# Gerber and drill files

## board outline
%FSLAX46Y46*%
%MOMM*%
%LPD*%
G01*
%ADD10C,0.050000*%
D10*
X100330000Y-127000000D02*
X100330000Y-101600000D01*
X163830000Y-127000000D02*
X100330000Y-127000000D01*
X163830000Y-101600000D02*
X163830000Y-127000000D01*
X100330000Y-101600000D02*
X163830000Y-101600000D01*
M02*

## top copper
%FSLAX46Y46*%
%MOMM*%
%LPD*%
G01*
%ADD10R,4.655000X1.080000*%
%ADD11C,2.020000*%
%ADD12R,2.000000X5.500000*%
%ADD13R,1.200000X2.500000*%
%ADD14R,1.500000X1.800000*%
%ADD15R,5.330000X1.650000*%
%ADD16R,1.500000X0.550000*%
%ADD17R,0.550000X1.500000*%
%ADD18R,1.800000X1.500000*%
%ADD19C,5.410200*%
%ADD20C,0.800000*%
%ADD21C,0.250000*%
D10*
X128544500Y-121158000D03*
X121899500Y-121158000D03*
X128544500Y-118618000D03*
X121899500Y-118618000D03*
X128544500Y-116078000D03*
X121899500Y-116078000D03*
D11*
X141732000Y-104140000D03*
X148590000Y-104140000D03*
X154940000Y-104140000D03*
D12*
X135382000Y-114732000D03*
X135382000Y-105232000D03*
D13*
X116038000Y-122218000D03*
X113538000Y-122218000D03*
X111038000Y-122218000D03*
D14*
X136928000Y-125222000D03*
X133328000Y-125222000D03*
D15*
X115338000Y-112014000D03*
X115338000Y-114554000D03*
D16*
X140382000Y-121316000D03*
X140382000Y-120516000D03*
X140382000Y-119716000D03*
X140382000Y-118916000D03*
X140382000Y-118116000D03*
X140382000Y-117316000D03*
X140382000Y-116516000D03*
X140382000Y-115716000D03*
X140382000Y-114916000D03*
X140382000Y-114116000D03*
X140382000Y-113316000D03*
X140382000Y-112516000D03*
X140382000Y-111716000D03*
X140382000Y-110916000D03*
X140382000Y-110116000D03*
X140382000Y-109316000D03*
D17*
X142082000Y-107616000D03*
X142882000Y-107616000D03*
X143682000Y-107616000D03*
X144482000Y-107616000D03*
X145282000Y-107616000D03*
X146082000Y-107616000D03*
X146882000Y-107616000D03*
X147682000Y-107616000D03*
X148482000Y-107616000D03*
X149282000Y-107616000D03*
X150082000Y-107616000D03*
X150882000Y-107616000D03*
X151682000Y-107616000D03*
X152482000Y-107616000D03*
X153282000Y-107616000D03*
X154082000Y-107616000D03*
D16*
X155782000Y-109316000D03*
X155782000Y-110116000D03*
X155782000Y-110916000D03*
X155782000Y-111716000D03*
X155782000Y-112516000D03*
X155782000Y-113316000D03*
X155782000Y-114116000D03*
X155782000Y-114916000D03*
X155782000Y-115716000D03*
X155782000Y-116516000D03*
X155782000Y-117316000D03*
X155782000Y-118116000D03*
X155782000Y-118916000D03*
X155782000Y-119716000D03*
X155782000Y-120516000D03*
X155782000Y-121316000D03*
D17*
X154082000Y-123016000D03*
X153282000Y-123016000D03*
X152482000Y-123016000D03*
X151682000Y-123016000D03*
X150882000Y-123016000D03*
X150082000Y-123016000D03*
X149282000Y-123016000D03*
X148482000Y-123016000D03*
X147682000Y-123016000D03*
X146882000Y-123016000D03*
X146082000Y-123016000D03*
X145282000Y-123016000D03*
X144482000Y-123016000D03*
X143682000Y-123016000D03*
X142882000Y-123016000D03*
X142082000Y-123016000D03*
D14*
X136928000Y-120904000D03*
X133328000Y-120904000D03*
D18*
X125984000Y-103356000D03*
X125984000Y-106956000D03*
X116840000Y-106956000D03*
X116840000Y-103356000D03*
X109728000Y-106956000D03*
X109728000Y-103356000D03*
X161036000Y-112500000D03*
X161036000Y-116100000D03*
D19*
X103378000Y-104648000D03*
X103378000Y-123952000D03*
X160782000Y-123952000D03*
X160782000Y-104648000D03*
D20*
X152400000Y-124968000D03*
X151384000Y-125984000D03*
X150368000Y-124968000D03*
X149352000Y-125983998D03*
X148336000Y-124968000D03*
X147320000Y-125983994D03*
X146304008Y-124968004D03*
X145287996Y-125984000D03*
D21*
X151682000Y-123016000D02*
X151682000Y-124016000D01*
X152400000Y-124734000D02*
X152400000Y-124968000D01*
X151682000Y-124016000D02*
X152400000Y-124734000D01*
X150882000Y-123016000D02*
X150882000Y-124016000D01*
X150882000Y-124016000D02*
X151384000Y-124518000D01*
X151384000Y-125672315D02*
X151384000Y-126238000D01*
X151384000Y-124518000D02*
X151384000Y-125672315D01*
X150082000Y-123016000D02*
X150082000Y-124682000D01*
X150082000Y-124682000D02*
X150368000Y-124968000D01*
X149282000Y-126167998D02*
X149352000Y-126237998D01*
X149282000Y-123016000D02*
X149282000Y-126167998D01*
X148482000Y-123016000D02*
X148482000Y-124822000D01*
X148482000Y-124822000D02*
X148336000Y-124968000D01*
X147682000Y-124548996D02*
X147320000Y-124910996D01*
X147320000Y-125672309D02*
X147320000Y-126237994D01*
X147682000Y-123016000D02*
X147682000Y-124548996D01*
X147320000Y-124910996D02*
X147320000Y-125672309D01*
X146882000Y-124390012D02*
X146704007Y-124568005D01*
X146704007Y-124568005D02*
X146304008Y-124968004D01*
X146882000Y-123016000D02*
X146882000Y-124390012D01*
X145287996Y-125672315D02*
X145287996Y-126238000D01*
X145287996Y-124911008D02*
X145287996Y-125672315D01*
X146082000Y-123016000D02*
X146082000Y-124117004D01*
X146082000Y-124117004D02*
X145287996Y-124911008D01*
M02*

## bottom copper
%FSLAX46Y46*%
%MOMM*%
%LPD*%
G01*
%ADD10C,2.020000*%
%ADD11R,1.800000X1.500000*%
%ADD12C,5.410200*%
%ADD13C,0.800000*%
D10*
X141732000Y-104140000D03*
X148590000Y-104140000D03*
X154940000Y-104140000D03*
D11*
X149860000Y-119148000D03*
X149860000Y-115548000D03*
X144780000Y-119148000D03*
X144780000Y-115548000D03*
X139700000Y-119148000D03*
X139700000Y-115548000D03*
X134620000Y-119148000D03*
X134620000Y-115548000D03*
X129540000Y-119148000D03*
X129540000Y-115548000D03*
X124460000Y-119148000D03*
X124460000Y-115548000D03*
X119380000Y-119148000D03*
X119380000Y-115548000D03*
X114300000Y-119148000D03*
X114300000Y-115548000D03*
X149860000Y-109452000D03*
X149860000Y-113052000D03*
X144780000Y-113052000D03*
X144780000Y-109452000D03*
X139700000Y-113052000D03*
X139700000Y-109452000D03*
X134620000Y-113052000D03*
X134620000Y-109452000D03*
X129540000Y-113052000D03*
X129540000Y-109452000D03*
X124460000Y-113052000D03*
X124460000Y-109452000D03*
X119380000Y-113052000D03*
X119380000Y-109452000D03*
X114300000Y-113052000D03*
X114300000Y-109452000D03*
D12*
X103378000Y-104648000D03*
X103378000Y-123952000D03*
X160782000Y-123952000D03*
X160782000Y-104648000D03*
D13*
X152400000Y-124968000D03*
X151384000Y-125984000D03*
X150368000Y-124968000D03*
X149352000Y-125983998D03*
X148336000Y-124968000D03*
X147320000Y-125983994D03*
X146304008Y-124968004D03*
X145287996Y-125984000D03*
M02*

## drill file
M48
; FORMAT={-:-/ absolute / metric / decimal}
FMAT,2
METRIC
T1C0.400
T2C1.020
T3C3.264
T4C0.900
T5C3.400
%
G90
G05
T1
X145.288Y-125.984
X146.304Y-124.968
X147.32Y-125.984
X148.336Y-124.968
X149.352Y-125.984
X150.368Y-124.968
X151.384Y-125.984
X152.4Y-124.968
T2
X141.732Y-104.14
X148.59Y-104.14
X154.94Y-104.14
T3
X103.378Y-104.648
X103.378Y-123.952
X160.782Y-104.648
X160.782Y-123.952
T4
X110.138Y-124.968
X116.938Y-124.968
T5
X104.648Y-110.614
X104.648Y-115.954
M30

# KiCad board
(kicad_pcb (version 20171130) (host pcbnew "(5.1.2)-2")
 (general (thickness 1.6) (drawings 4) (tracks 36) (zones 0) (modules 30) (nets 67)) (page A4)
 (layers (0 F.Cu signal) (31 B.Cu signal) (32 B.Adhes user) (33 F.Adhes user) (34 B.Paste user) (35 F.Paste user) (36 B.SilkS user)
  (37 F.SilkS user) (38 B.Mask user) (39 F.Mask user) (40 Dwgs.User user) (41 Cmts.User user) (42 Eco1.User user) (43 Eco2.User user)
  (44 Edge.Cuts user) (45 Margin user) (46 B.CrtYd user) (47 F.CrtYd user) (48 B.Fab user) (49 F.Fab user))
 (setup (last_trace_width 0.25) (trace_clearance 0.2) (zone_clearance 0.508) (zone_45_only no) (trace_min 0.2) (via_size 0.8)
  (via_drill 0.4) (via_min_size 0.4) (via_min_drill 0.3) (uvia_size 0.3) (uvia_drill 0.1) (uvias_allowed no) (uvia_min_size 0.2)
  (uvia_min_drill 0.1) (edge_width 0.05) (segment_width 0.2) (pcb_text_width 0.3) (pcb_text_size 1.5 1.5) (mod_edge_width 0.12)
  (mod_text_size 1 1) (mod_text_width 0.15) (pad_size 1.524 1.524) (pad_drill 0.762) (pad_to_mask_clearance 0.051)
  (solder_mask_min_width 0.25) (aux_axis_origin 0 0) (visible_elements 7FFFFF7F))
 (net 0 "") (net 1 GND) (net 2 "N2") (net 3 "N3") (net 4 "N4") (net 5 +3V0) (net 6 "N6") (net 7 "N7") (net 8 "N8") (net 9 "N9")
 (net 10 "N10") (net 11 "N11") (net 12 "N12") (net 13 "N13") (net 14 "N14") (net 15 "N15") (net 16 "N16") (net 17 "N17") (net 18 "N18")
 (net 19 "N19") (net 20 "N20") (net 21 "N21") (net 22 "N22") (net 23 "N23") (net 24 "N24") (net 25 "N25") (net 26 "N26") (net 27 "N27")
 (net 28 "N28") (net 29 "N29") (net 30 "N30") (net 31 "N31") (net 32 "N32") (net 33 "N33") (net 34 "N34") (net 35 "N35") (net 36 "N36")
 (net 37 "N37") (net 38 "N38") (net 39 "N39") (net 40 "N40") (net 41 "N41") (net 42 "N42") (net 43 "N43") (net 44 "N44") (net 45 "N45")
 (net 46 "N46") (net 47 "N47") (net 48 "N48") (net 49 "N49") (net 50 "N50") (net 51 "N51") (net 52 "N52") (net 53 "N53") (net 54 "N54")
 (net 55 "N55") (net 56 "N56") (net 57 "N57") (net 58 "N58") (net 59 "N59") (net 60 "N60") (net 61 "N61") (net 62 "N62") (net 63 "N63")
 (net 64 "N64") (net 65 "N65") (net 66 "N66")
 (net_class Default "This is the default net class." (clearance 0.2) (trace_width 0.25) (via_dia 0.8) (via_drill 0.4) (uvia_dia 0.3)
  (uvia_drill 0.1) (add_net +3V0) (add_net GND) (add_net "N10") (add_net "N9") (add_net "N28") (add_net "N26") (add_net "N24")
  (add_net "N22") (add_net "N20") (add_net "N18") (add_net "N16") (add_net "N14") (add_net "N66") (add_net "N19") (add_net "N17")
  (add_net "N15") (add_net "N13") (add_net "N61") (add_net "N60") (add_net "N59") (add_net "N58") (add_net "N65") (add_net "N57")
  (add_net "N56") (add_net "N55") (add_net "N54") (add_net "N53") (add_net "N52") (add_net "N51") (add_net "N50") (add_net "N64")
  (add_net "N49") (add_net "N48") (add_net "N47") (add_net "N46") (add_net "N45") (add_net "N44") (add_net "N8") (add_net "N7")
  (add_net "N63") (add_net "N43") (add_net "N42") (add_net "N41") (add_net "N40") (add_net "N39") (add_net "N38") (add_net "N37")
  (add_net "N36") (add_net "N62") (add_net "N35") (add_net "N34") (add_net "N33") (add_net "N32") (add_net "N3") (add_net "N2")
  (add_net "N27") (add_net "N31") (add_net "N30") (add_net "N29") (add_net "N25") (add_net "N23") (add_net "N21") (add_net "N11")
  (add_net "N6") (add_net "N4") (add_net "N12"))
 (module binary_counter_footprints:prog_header (layer F.Cu) (at 125.222 118.618 90)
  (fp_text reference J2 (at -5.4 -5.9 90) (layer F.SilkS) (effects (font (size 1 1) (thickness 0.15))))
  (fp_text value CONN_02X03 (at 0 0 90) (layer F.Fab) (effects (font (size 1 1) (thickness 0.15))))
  (pad 6 smd rect (at -2.54 3.3225 90) (size 1.08 4.655) (layers F.Cu F.Paste F.Mask) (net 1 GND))
  (pad 5 smd rect (at -2.54 -3.3225 90) (size 1.08 4.655) (layers F.Cu F.Paste F.Mask) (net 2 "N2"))
  (pad 4 smd rect (at 0 3.3225 90) (size 1.08 4.655) (layers F.Cu F.Paste F.Mask) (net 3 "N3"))
  (pad 3 smd rect (at 0 -3.3225 90) (size 1.08 4.655) (layers F.Cu F.Paste F.Mask) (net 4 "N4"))
  (pad 2 smd rect (at 2.54 3.3225 90) (size 1.08 4.655) (layers F.Cu F.Paste F.Mask) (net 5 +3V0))
  (pad 1 smd rect (at 2.54 -3.3225 90) (size 1.08 4.655) (layers F.Cu F.Paste F.Mask) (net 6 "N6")))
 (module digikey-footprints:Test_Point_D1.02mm (layer F.Cu) (at 141.732 104.14)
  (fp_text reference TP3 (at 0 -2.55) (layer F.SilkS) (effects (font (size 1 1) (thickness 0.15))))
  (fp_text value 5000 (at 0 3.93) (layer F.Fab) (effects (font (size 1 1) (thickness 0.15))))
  (pad 1 thru_hole circle (at 0 0) (size 2.02 2.02) (drill 1.02) (layers *.Cu *.Mask) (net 1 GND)))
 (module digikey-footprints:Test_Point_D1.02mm (layer F.Cu) (at 148.59 104.14)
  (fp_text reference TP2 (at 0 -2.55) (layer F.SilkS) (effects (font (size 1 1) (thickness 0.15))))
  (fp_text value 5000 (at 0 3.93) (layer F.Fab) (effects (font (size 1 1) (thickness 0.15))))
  (pad 1 thru_hole circle (at 0 0) (size 2.02 2.02) (drill 1.02) (layers *.Cu *.Mask) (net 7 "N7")))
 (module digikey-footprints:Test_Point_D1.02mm (layer F.Cu) (at 154.94 104.14)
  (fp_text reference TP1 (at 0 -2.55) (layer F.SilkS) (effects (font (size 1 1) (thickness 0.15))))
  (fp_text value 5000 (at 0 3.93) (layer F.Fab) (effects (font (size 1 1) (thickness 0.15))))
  (pad 1 thru_hole circle (at 0 0) (size 2.02 2.02) (drill 1.02) (layers *.Cu *.Mask) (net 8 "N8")))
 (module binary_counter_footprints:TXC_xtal (layer F.Cu) (at 135.382 109.982 270)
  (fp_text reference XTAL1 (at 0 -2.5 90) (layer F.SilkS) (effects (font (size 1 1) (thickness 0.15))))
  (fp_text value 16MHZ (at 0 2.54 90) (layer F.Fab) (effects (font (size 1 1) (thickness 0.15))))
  (pad 2 smd rect (at 4.75 0 270) (size 5.5 2) (layers F.Cu F.Paste F.Mask) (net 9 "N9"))
  (pad 1 smd rect (at -4.75 0 270) (size 5.5 2) (layers F.Cu F.Paste F.Mask) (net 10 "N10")))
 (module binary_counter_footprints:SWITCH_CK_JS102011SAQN (layer F.Cu) (at 113.538 124.968)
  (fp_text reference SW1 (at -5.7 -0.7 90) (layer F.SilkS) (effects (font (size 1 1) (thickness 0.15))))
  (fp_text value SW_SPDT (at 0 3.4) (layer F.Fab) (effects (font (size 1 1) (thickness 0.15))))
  (pad "" np_thru_hole circle (at 3.4 0) (size 0.9 0.9) (drill 0.9) (layers *.Cu *.Mask))
  (pad "" np_thru_hole circle (at -3.4 0) (size 0.9 0.9) (drill 0.9) (layers *.Cu *.Mask))
  (pad 3 smd rect (at 2.5 -2.75) (size 1.2 2.5) (layers F.Cu F.Paste F.Mask) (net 5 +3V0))
  (pad 2 smd rect (at 0 -2.75) (size 1.2 2.5) (layers F.Cu F.Paste F.Mask) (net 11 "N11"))
  (pad 1 smd rect (at -2.5 -2.75) (size 1.2 2.5) (layers F.Cu F.Paste F.Mask) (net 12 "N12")))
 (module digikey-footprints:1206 (layer B.Cu) (at 149.86 117.348 270)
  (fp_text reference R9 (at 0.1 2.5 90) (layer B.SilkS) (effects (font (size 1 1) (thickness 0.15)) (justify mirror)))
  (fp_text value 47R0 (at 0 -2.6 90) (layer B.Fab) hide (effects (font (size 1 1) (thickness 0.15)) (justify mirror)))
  (pad 2 smd rect (at 1.8 0 270) (size 1.5 1.8) (layers B.Cu B.Paste B.Mask) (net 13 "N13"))
  (pad 1 smd rect (at -1.8 0 270) (size 1.5 1.8) (layers B.Cu B.Paste B.Mask) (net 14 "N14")))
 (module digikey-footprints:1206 (layer B.Cu) (at 144.78 117.348 270)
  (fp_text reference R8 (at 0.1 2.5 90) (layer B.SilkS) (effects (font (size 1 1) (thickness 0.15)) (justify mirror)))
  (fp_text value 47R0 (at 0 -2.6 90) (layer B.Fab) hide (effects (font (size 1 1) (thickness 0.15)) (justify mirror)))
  (pad 2 smd rect (at 1.8 0 270) (size 1.5 1.8) (layers B.Cu B.Paste B.Mask) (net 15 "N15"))
  (pad 1 smd rect (at -1.8 0 270) (size 1.5 1.8) (layers B.Cu B.Paste B.Mask) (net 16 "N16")))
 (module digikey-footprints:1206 (layer B.Cu) (at 139.7 117.348 270)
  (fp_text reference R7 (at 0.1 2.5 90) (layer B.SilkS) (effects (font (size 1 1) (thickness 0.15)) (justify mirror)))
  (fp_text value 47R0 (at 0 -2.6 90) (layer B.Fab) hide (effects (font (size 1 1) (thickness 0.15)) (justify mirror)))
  (pad 2 smd rect (at 1.8 0 270) (size 1.5 1.8) (layers B.Cu B.Paste B.Mask) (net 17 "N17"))
  (pad 1 smd rect (at -1.8 0 270) (size 1.5 1.8) (layers B.Cu B.Paste B.Mask) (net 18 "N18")))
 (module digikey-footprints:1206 (layer B.Cu) (at 134.62 117.348 270)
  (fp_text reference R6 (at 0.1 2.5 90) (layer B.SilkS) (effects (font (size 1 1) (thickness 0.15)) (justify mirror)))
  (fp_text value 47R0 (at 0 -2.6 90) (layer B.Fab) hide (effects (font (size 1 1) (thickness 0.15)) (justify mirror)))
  (pad 2 smd rect (at 1.8 0 270) (size 1.5 1.8) (layers B.Cu B.Paste B.Mask) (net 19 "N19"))
  (pad 1 smd rect (at -1.8 0 270) (size 1.5 1.8) (layers B.Cu B.Paste B.Mask) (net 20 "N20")))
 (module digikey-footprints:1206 (layer B.Cu) (at 129.54 117.348 270)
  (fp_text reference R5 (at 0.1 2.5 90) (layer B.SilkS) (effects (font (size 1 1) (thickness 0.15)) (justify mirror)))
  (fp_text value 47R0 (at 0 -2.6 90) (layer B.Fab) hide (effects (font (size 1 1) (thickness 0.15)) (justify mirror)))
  (pad 2 smd rect (at 1.8 0 270) (size 1.5 1.8) (layers B.Cu B.Paste B.Mask) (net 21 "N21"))
  (pad 1 smd rect (at -1.8 0 270) (size 1.5 1.8) (layers B.Cu B.Paste B.Mask) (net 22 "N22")))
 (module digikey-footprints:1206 (layer B.Cu) (at 124.46 117.348 270)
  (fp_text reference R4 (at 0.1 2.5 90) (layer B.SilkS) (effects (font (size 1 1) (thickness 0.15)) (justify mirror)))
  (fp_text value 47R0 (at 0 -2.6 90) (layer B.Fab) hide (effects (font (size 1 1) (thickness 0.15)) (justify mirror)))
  (pad 2 smd rect (at 1.8 0 270) (size 1.5 1.8) (layers B.Cu B.Paste B.Mask) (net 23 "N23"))
  (pad 1 smd rect (at -1.8 0 270) (size 1.5 1.8) (layers B.Cu B.Paste B.Mask) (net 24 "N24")))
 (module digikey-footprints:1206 (layer B.Cu) (at 119.38 117.348 270)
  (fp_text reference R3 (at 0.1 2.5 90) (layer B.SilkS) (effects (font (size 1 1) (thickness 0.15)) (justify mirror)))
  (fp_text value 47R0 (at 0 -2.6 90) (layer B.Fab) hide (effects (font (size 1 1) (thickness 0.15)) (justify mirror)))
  (pad 2 smd rect (at 1.8 0 270) (size 1.5 1.8) (layers B.Cu B.Paste B.Mask) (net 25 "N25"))
  (pad 1 smd rect (at -1.8 0 270) (size 1.5 1.8) (layers B.Cu B.Paste B.Mask) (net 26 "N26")))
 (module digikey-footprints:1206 (layer B.Cu) (at 114.3 117.348 270)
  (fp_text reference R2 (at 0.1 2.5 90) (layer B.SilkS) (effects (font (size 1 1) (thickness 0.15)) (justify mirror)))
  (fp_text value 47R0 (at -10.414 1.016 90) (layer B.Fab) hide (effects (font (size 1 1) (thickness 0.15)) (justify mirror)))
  (pad 2 smd rect (at 1.8 0 270) (size 1.5 1.8) (layers B.Cu B.Paste B.Mask) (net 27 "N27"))
  (pad 1 smd rect (at -1.8 0 270) (size 1.5 1.8) (layers B.Cu B.Paste B.Mask) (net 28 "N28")))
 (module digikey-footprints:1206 (layer F.Cu) (at 135.128 125.222)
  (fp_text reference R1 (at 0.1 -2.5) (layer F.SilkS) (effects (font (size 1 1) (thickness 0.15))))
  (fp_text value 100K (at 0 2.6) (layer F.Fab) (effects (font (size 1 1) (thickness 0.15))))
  (pad 2 smd rect (at 1.8 0) (size 1.5 1.8) (layers F.Cu F.Paste F.Mask) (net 5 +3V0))
  (pad 1 smd rect (at -1.8 0) (size 1.5 1.8) (layers F.Cu F.Paste F.Mask) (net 2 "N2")))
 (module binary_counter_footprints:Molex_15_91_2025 (layer F.Cu) (at 104.648 113.284 270)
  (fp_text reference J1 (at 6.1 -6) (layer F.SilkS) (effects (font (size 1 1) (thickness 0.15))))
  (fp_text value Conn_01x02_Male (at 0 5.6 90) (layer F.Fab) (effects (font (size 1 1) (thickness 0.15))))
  (pad "" np_thru_hole circle (at -2.67 0 270) (size 3.4 3.4) (drill 3.4) (layers *.Cu *.Mask))
  (pad "" np_thru_hole circle (at 2.67 0 270) (size 3.4 3.4) (drill 3.4) (layers *.Cu *.Mask))
  (pad 2 smd rect (at -1.27 -10.69 270) (size 1.65 5.33) (layers F.Cu F.Paste F.Mask) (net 1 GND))
  (pad 1 smd rect (at 1.27 -10.69 270) (size 1.65 5.33) (layers F.Cu F.Paste F.Mask) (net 11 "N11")))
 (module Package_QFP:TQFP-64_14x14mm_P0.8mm (layer F.Cu) (at 148.082 115.316 90)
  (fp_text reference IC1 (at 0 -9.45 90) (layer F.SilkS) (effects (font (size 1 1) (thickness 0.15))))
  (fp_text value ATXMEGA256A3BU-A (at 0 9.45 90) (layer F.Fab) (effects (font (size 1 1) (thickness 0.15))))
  (pad 64 smd rect (at -6 -7.7 180) (size 1.5 0.55) (layers F.Cu F.Paste F.Mask) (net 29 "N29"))
  (pad 63 smd rect (at -5.2 -7.7 180) (size 1.5 0.55) (layers F.Cu F.Paste F.Mask) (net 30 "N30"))
  (pad 62 smd rect (at -4.4 -7.7 180) (size 1.5 0.55) (layers F.Cu F.Paste F.Mask) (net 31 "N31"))
  (pad 61 smd rect (at -3.6 -7.7 180) (size 1.5 0.55) (layers F.Cu F.Paste F.Mask) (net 5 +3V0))
  (pad 60 smd rect (at -2.8 -7.7 180) (size 1.5 0.55) (layers F.Cu F.Paste F.Mask) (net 1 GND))
  (pad 59 smd rect (at -2 -7.7 180) (size 1.5 0.55) (layers F.Cu F.Paste F.Mask) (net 9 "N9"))
  (pad 58 smd rect (at -1.2 -7.7 180) (size 1.5 0.55) (layers F.Cu F.Paste F.Mask) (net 10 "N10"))
  (pad 57 smd rect (at -0.4 -7.7 180) (size 1.5 0.55) (layers F.Cu F.Paste F.Mask) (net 2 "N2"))
  (pad 56 smd rect (at 0.4 -7.7 180) (size 1.5 0.55) (layers F.Cu F.Paste F.Mask) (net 3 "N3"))
  (pad 55 smd rect (at 1.2 -7.7 180) (size 1.5 0.55) (layers F.Cu F.Paste F.Mask) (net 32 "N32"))
  (pad 54 smd rect (at 2 -7.7 180) (size 1.5 0.55) (layers F.Cu F.Paste F.Mask) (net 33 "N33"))
  (pad 53 smd rect (at 2.8 -7.7 180) (size 1.5 0.55) (layers F.Cu F.Paste F.Mask) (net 5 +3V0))
  (pad 52 smd rect (at 3.6 -7.7 180) (size 1.5 0.55) (layers F.Cu F.Paste F.Mask) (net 1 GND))
  (pad 51 smd rect (at 4.4 -7.7 180) (size 1.5 0.55) (layers F.Cu F.Paste F.Mask) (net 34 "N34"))
  (pad 50 smd rect (at 5.2 -7.7 180) (size 1.5 0.55) (layers F.Cu F.Paste F.Mask) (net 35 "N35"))
  (pad 49 smd rect (at 6 -7.7 180) (size 1.5 0.55) (layers F.Cu F.Paste F.Mask) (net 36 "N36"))
  (pad 48 smd rect (at 7.7 -6 90) (size 1.5 0.55) (layers F.Cu F.Paste F.Mask) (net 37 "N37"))
  (pad 47 smd rect (at 7.7 -5.2 90) (size 1.5 0.55) (layers F.Cu F.Paste F.Mask) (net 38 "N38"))
  (pad 46 smd rect (at 7.7 -4.4 90) (size 1.5 0.55) (layers F.Cu F.Paste F.Mask) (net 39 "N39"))
  (pad 45 smd rect (at 7.7 -3.6 90) (size 1.5 0.55) (layers F.Cu F.Paste F.Mask) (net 5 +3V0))
  (pad 44 smd rect (at 7.7 -2.8 90) (size 1.5 0.55) (layers F.Cu F.Paste F.Mask) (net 1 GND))
  (pad 43 smd rect (at 7.7 -2 90) (size 1.5 0.55) (layers F.Cu F.Paste F.Mask) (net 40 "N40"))
  (pad 42 smd rect (at 7.7 -1.2 90) (size 1.5 0.55) (layers F.Cu F.Paste F.Mask) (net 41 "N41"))
  (pad 41 smd rect (at 7.7 -0.4 90) (size 1.5 0.55) (layers F.Cu F.Paste F.Mask) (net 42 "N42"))
  (pad 40 smd rect (at 7.7 0.4 90) (size 1.5 0.55) (layers F.Cu F.Paste F.Mask) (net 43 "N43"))
  (pad 39 smd rect (at 7.7 1.2 90) (size 1.5 0.55) (layers F.Cu F.Paste F.Mask) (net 7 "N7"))
  (pad 38 smd rect (at 7.7 2 90) (size 1.5 0.55) (layers F.Cu F.Paste F.Mask) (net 8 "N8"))
  (pad 37 smd rect (at 7.7 2.8 90) (size 1.5 0.55) (layers F.Cu F.Paste F.Mask) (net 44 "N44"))
  (pad 36 smd rect (at 7.7 3.6 90) (size 1.5 0.55) (layers F.Cu F.Paste F.Mask) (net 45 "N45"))
  (pad 35 smd rect (at 7.7 4.4 90) (size 1.5 0.55) (layers F.Cu F.Paste F.Mask) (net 5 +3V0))
  (pad 34 smd rect (at 7.7 5.2 90) (size 1.5 0.55) (layers F.Cu F.Paste F.Mask) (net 1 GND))
  (pad 33 smd rect (at 7.7 6 90) (size 1.5 0.55) (layers F.Cu F.Paste F.Mask) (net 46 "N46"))
  (pad 32 smd rect (at 6 7.7 180) (size 1.5 0.55) (layers F.Cu F.Paste F.Mask) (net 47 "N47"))
  (pad 31 smd rect (at 5.2 7.7 180) (size 1.5 0.55) (layers F.Cu F.Paste F.Mask) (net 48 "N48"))
  (pad 30 smd rect (at 4.4 7.7 180) (size 1.5 0.55) (layers F.Cu F.Paste F.Mask) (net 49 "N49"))
  (pad 29 smd rect (at 3.6 7.7 180) (size 1.5 0.55) (layers F.Cu F.Paste F.Mask) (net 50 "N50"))
  (pad 28 smd rect (at 2.8 7.7 180) (size 1.5 0.55) (layers F.Cu F.Paste F.Mask) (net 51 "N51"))
  (pad 27 smd rect (at 2 7.7 180) (size 1.5 0.55) (layers F.Cu F.Paste F.Mask) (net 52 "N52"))
  (pad 26 smd rect (at 1.2 7.7 180) (size 1.5 0.55) (layers F.Cu F.Paste F.Mask) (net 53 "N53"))
  (pad 25 smd rect (at 0.4 7.7 180) (size 1.5 0.55) (layers F.Cu F.Paste F.Mask) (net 5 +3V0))
  (pad 24 smd rect (at -0.4 7.7 180) (size 1.5 0.55) (layers F.Cu F.Paste F.Mask) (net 1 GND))
  (pad 23 smd rect (at -1.2 7.7 180) (size 1.5 0.55) (layers F.Cu F.Paste F.Mask) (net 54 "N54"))
  (pad 22 smd rect (at -2 7.7 180) (size 1.5 0.55) (layers F.Cu F.Paste F.Mask) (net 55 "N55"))
  (pad 21 smd rect (at -2.8 7.7 180) (size 1.5 0.55) (layers F.Cu F.Paste F.Mask) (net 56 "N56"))
  (pad 20 smd rect (at -3.6 7.7 180) (size 1.5 0.55) (layers F.Cu F.Paste F.Mask) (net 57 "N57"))
  (pad 19 smd rect (at -4.4 7.7 180) (size 1.5 0.55) (layers F.Cu F.Paste F.Mask) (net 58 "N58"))
  (pad 18 smd rect (at -5.2 7.7 180) (size 1.5 0.55) (layers F.Cu F.Paste F.Mask) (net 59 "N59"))
  (pad 17 smd rect (at -6 7.7 180) (size 1.5 0.55) (layers F.Cu F.Paste F.Mask) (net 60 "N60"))
  (pad 16 smd rect (at -7.7 6 90) (size 1.5 0.55) (layers F.Cu F.Paste F.Mask) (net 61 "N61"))
  (pad 15 smd rect (at -7.7 5.2 90) (size 1.5 0.55) (layers F.Cu F.Paste F.Mask) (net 5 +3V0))
  (pad 14 smd rect (at -7.7 4.4 90) (size 1.5 0.55) (layers F.Cu F.Paste F.Mask) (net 1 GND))
  (pad 13 smd rect (at -7.7 3.6 90) (size 1.5 0.55) (layers F.Cu F.Paste F.Mask) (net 13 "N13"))
  (pad 12 smd rect (at -7.7 2.8 90) (size 1.5 0.55) (layers F.Cu F.Paste F.Mask) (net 15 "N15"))
  (pad 11 smd rect (at -7.7 2 90) (size 1.5 0.55) (layers F.Cu F.Paste F.Mask) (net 17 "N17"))
  (pad 10 smd rect (at -7.7 1.2 90) (size 1.5 0.55) (layers F.Cu F.Paste F.Mask) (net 19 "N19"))
  (pad 9 smd rect (at -7.7 0.4 90) (size 1.5 0.55) (layers F.Cu F.Paste F.Mask) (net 21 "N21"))
  (pad 8 smd rect (at -7.7 -0.4 90) (size 1.5 0.55) (layers F.Cu F.Paste F.Mask) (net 23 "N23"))
  (pad 7 smd rect (at -7.7 -1.2 90) (size 1.5 0.55) (layers F.Cu F.Paste F.Mask) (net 25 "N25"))
  (pad 6 smd rect (at -7.7 -2 90) (size 1.5 0.55) (layers F.Cu F.Paste F.Mask) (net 27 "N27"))
  (pad 5 smd rect (at -7.7 -2.8 90) (size 1.5 0.55) (layers F.Cu F.Paste F.Mask) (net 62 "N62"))
  (pad 4 smd rect (at -7.7 -3.6 90) (size 1.5 0.55) (layers F.Cu F.Paste F.Mask) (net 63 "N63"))
  (pad 3 smd rect (at -7.7 -4.4 90) (size 1.5 0.55) (layers F.Cu F.Paste F.Mask) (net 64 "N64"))
  (pad 2 smd rect (at -7.7 -5.2 90) (size 1.5 0.55) (layers F.Cu F.Paste F.Mask) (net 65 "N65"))
  (pad 1 smd rect (at -7.7 -6 90) (size 1.5 0.55) (layers F.Cu F.Paste F.Mask) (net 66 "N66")))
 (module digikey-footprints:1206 (layer B.Cu) (at 149.86 111.252 270)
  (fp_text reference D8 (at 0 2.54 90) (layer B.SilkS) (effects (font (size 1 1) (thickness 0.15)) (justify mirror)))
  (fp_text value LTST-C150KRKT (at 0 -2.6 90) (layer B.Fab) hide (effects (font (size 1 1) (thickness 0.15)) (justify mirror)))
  (pad 1 smd rect (at -1.8 0 270) (size 1.5 1.8) (layers B.Cu B.Paste B.Mask) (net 5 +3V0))
  (pad 2 smd rect (at 1.8 0 270) (size 1.5 1.8) (layers B.Cu B.Paste B.Mask) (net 14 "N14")))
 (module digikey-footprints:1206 (layer B.Cu) (at 144.78 111.252 270)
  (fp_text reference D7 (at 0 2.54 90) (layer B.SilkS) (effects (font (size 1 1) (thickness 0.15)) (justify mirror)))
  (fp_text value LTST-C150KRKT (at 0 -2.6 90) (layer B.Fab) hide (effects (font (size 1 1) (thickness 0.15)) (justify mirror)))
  (pad 2 smd rect (at 1.8 0 270) (size 1.5 1.8) (layers B.Cu B.Paste B.Mask) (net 16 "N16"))
  (pad 1 smd rect (at -1.8 0 270) (size 1.5 1.8) (layers B.Cu B.Paste B.Mask) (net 5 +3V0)))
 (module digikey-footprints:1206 (layer B.Cu) (at 139.7 111.252 270)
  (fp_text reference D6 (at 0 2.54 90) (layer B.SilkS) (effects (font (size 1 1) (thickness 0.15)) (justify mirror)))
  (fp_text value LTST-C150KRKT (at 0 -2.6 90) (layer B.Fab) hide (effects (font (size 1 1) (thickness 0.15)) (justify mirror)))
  (pad 2 smd rect (at 1.8 0 270) (size 1.5 1.8) (layers B.Cu B.Paste B.Mask) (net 18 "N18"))
  (pad 1 smd rect (at -1.8 0 270) (size 1.5 1.8) (layers B.Cu B.Paste B.Mask) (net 5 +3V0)))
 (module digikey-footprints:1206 (layer B.Cu) (at 134.62 111.252 270)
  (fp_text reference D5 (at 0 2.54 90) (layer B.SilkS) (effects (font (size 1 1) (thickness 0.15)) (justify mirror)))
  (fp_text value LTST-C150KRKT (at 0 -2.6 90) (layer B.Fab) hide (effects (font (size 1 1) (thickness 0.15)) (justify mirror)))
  (pad 2 smd rect (at 1.8 0 270) (size 1.5 1.8) (layers B.Cu B.Paste B.Mask) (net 20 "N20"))
  (pad 1 smd rect (at -1.8 0 270) (size 1.5 1.8) (layers B.Cu B.Paste B.Mask) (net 5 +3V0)))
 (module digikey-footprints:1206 (layer B.Cu) (at 129.54 111.252 270)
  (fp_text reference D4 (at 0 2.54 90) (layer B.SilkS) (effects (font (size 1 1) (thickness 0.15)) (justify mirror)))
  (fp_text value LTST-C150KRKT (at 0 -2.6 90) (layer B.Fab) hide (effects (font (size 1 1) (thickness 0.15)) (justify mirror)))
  (pad 2 smd rect (at 1.8 0 270) (size 1.5 1.8) (layers B.Cu B.Paste B.Mask) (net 22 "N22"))
  (pad 1 smd rect (at -1.8 0 270) (size 1.5 1.8) (layers B.Cu B.Paste B.Mask) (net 5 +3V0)))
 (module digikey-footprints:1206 (layer B.Cu) (at 124.46 111.252 270)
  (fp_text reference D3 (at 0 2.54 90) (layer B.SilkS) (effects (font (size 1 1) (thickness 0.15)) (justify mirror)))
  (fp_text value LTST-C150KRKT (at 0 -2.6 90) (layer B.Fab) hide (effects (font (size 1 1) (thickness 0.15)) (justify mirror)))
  (pad 2 smd rect (at 1.8 0 270) (size 1.5 1.8) (layers B.Cu B.Paste B.Mask) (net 24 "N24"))
  (pad 1 smd rect (at -1.8 0 270) (size 1.5 1.8) (layers B.Cu B.Paste B.Mask) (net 5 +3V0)))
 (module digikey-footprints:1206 (layer B.Cu) (at 119.38 111.252 270)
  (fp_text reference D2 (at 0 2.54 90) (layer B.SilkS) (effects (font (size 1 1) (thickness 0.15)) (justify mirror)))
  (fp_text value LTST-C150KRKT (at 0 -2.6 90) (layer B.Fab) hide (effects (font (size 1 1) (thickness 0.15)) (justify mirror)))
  (pad 2 smd rect (at 1.8 0 270) (size 1.5 1.8) (layers B.Cu B.Paste B.Mask) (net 26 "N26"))
  (pad 1 smd rect (at -1.8 0 270) (size 1.5 1.8) (layers B.Cu B.Paste B.Mask) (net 5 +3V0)))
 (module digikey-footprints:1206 (layer B.Cu) (at 114.3 111.252 270)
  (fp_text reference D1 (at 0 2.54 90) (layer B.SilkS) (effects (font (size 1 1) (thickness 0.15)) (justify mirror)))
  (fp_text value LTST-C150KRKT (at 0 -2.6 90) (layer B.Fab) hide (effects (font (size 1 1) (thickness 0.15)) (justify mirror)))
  (pad 2 smd rect (at 1.8 0 270) (size 1.5 1.8) (layers B.Cu B.Paste B.Mask) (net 28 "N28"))
  (pad 1 smd rect (at -1.8 0 270) (size 1.5 1.8) (layers B.Cu B.Paste B.Mask) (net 5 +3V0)))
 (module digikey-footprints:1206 (layer F.Cu) (at 135.128 120.904)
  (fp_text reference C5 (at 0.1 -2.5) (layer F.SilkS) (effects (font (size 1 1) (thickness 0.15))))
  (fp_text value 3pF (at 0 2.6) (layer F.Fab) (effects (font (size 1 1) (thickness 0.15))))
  (pad 2 smd rect (at 1.8 0) (size 1.5 1.8) (layers F.Cu F.Paste F.Mask) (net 9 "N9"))
  (pad 1 smd rect (at -1.8 0) (size 1.5 1.8) (layers F.Cu F.Paste F.Mask) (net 1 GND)))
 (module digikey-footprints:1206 (layer F.Cu) (at 125.984 105.156 90)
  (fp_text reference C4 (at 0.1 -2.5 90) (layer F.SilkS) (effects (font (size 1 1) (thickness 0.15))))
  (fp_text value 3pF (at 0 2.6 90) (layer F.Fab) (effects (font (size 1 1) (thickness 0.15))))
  (pad 2 smd rect (at 1.8 0 90) (size 1.5 1.8) (layers F.Cu F.Paste F.Mask) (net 10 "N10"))
  (pad 1 smd rect (at -1.8 0 90) (size 1.5 1.8) (layers F.Cu F.Paste F.Mask) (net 1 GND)))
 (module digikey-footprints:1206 (layer F.Cu) (at 116.84 105.156 270)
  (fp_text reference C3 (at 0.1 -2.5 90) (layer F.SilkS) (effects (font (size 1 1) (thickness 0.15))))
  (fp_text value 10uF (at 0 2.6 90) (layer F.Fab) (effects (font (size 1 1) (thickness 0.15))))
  (pad 2 smd rect (at 1.8 0 270) (size 1.5 1.8) (layers F.Cu F.Paste F.Mask) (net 1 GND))
  (pad 1 smd rect (at -1.8 0 270) (size 1.5 1.8) (layers F.Cu F.Paste F.Mask) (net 5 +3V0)))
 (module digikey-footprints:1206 (layer F.Cu) (at 109.728 105.156 270)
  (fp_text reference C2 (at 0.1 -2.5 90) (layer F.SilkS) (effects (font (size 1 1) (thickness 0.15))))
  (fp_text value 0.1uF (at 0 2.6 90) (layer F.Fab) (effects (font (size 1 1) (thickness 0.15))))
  (pad 2 smd rect (at 1.8 0 270) (size 1.5 1.8) (layers F.Cu F.Paste F.Mask) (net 1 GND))
  (pad 1 smd rect (at -1.8 0 270) (size 1.5 1.8) (layers F.Cu F.Paste F.Mask) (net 5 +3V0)))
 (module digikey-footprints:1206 (layer F.Cu) (at 161.036 114.3 90)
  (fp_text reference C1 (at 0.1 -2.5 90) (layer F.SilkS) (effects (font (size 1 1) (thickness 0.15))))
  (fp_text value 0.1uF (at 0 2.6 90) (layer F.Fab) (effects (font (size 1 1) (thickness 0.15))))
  (pad 2 smd rect (at 1.8 0 90) (size 1.5 1.8) (layers F.Cu F.Paste F.Mask) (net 1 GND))
  (pad 1 smd rect (at -1.8 0 90) (size 1.5 1.8) (layers F.Cu F.Paste F.Mask) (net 5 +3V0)))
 (gr_line (start 100.33 127) (end 100.33 101.6) (layer Edge.Cuts) (width 0.05))
 (gr_line (start 163.83 127) (end 100.33 127) (layer Edge.Cuts) (width 0.05))
 (gr_line (start 163.83 101.6) (end 163.83 127) (layer Edge.Cuts) (width 0.05))
 (gr_line (start 100.33 101.6) (end 163.83 101.6) (layer Edge.Cuts) (width 0.05))
 (via (at 103.378 104.648) (size 5.4102) (drill 3.2639) (layers F.Cu B.Cu) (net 1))
 (via (at 103.378 123.952) (size 5.4102) (drill 3.2639) (layers F.Cu B.Cu) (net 1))
 (via (at 160.782 123.952) (size 5.4102) (drill 3.2639) (layers F.Cu B.Cu) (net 1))
 (via (at 160.782 104.648) (size 5.4102) (drill 3.2639) (layers F.Cu B.Cu) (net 1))
 (via (at 152.4 124.968) (size 0.8) (drill 0.4) (layers F.Cu B.Cu) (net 13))
 (segment (start 151.682 123.016) (end 151.682 124.016) (width 0.25) (layer F.Cu) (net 13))
 (segment (start 152.4 124.734) (end 152.4 124.968) (width 0.25) (layer F.Cu) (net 13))
 (segment (start 151.682 124.016) (end 152.4 124.734) (width 0.25) (layer F.Cu) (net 13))
 (via (at 151.384 125.984) (size 0.8) (drill 0.4) (layers F.Cu B.Cu) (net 15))
 (segment (start 150.882 123.016) (end 150.882 124.016) (width 0.25) (layer F.Cu) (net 15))
 (segment (start 150.882 124.016) (end 151.384 124.518) (width 0.25) (layer F.Cu) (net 15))
 (segment (start 151.384 125.672315) (end 151.384 126.238) (width 0.25) (layer F.Cu) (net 15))
 (segment (start 151.384 124.518) (end 151.384 125.672315) (width 0.25) (layer F.Cu) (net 15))
 (via (at 150.368 124.968) (size 0.8) (drill 0.4) (layers F.Cu B.Cu) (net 17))
 (segment (start 150.082 123.016) (end 150.082 124.682) (width 0.25) (layer F.Cu) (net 17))
 (segment (start 150.082 124.682) (end 150.368 124.968) (width 0.25) (layer F.Cu) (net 17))
 (via (at 149.352 125.983998) (size 0.8) (drill 0.4) (layers F.Cu B.Cu) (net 19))
 (segment (start 149.282 126.167998) (end 149.352 126.237998) (width 0.25) (layer F.Cu) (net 19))
 (segment (start 149.282 123.016) (end 149.282 126.167998) (width 0.25) (layer F.Cu) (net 19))
 (segment (start 148.482 123.016) (end 148.482 124.822) (width 0.25) (layer F.Cu) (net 21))
 (segment (start 148.482 124.822) (end 148.336 124.968) (width 0.25) (layer F.Cu) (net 21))
 (via (at 148.336 124.968) (size 0.8) (drill 0.4) (layers F.Cu B.Cu) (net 21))
 (via (at 147.32 125.983994) (size 0.8) (drill 0.4) (layers F.Cu B.Cu) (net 23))
 (segment (start 147.682 124.548996) (end 147.32 124.910996) (width 0.25) (layer F.Cu) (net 23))
 (segment (start 147.32 125.672309) (end 147.32 126.237994) (width 0.25) (layer F.Cu) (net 23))
 (segment (start 147.682 123.016) (end 147.682 124.548996) (width 0.25) (layer F.Cu) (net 23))
 (segment (start 147.32 124.910996) (end 147.32 125.672309) (width 0.25) (layer F.Cu) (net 23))
 (segment (start 146.882 124.390012) (end 146.704007 124.568005) (width 0.25) (layer F.Cu) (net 25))
 (segment (start 146.704007 124.568005) (end 146.304008 124.968004) (width 0.25) (layer F.Cu) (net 25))
 (segment (start 146.882 123.016) (end 146.882 124.390012) (width 0.25) (layer F.Cu) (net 25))
 (via (at 146.304008 124.968004) (size 0.8) (drill 0.4) (layers F.Cu B.Cu) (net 25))
 (via (at 145.287996 125.984) (size 0.8) (drill 0.4) (layers F.Cu B.Cu) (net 27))
 (segment (start 145.287996 125.672315) (end 145.287996 126.238) (width 0.25) (layer F.Cu) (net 27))
 (segment (start 145.287996 124.911008) (end 145.287996 125.672315) (width 0.25) (layer F.Cu) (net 27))
 (segment (start 146.082 123.016) (end 146.082 124.117004) (width 0.25) (layer F.Cu) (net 27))
 (segment (start 146.082 124.117004) (end 145.287996 124.911008) (width 0.25) (layer F.Cu) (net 27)))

